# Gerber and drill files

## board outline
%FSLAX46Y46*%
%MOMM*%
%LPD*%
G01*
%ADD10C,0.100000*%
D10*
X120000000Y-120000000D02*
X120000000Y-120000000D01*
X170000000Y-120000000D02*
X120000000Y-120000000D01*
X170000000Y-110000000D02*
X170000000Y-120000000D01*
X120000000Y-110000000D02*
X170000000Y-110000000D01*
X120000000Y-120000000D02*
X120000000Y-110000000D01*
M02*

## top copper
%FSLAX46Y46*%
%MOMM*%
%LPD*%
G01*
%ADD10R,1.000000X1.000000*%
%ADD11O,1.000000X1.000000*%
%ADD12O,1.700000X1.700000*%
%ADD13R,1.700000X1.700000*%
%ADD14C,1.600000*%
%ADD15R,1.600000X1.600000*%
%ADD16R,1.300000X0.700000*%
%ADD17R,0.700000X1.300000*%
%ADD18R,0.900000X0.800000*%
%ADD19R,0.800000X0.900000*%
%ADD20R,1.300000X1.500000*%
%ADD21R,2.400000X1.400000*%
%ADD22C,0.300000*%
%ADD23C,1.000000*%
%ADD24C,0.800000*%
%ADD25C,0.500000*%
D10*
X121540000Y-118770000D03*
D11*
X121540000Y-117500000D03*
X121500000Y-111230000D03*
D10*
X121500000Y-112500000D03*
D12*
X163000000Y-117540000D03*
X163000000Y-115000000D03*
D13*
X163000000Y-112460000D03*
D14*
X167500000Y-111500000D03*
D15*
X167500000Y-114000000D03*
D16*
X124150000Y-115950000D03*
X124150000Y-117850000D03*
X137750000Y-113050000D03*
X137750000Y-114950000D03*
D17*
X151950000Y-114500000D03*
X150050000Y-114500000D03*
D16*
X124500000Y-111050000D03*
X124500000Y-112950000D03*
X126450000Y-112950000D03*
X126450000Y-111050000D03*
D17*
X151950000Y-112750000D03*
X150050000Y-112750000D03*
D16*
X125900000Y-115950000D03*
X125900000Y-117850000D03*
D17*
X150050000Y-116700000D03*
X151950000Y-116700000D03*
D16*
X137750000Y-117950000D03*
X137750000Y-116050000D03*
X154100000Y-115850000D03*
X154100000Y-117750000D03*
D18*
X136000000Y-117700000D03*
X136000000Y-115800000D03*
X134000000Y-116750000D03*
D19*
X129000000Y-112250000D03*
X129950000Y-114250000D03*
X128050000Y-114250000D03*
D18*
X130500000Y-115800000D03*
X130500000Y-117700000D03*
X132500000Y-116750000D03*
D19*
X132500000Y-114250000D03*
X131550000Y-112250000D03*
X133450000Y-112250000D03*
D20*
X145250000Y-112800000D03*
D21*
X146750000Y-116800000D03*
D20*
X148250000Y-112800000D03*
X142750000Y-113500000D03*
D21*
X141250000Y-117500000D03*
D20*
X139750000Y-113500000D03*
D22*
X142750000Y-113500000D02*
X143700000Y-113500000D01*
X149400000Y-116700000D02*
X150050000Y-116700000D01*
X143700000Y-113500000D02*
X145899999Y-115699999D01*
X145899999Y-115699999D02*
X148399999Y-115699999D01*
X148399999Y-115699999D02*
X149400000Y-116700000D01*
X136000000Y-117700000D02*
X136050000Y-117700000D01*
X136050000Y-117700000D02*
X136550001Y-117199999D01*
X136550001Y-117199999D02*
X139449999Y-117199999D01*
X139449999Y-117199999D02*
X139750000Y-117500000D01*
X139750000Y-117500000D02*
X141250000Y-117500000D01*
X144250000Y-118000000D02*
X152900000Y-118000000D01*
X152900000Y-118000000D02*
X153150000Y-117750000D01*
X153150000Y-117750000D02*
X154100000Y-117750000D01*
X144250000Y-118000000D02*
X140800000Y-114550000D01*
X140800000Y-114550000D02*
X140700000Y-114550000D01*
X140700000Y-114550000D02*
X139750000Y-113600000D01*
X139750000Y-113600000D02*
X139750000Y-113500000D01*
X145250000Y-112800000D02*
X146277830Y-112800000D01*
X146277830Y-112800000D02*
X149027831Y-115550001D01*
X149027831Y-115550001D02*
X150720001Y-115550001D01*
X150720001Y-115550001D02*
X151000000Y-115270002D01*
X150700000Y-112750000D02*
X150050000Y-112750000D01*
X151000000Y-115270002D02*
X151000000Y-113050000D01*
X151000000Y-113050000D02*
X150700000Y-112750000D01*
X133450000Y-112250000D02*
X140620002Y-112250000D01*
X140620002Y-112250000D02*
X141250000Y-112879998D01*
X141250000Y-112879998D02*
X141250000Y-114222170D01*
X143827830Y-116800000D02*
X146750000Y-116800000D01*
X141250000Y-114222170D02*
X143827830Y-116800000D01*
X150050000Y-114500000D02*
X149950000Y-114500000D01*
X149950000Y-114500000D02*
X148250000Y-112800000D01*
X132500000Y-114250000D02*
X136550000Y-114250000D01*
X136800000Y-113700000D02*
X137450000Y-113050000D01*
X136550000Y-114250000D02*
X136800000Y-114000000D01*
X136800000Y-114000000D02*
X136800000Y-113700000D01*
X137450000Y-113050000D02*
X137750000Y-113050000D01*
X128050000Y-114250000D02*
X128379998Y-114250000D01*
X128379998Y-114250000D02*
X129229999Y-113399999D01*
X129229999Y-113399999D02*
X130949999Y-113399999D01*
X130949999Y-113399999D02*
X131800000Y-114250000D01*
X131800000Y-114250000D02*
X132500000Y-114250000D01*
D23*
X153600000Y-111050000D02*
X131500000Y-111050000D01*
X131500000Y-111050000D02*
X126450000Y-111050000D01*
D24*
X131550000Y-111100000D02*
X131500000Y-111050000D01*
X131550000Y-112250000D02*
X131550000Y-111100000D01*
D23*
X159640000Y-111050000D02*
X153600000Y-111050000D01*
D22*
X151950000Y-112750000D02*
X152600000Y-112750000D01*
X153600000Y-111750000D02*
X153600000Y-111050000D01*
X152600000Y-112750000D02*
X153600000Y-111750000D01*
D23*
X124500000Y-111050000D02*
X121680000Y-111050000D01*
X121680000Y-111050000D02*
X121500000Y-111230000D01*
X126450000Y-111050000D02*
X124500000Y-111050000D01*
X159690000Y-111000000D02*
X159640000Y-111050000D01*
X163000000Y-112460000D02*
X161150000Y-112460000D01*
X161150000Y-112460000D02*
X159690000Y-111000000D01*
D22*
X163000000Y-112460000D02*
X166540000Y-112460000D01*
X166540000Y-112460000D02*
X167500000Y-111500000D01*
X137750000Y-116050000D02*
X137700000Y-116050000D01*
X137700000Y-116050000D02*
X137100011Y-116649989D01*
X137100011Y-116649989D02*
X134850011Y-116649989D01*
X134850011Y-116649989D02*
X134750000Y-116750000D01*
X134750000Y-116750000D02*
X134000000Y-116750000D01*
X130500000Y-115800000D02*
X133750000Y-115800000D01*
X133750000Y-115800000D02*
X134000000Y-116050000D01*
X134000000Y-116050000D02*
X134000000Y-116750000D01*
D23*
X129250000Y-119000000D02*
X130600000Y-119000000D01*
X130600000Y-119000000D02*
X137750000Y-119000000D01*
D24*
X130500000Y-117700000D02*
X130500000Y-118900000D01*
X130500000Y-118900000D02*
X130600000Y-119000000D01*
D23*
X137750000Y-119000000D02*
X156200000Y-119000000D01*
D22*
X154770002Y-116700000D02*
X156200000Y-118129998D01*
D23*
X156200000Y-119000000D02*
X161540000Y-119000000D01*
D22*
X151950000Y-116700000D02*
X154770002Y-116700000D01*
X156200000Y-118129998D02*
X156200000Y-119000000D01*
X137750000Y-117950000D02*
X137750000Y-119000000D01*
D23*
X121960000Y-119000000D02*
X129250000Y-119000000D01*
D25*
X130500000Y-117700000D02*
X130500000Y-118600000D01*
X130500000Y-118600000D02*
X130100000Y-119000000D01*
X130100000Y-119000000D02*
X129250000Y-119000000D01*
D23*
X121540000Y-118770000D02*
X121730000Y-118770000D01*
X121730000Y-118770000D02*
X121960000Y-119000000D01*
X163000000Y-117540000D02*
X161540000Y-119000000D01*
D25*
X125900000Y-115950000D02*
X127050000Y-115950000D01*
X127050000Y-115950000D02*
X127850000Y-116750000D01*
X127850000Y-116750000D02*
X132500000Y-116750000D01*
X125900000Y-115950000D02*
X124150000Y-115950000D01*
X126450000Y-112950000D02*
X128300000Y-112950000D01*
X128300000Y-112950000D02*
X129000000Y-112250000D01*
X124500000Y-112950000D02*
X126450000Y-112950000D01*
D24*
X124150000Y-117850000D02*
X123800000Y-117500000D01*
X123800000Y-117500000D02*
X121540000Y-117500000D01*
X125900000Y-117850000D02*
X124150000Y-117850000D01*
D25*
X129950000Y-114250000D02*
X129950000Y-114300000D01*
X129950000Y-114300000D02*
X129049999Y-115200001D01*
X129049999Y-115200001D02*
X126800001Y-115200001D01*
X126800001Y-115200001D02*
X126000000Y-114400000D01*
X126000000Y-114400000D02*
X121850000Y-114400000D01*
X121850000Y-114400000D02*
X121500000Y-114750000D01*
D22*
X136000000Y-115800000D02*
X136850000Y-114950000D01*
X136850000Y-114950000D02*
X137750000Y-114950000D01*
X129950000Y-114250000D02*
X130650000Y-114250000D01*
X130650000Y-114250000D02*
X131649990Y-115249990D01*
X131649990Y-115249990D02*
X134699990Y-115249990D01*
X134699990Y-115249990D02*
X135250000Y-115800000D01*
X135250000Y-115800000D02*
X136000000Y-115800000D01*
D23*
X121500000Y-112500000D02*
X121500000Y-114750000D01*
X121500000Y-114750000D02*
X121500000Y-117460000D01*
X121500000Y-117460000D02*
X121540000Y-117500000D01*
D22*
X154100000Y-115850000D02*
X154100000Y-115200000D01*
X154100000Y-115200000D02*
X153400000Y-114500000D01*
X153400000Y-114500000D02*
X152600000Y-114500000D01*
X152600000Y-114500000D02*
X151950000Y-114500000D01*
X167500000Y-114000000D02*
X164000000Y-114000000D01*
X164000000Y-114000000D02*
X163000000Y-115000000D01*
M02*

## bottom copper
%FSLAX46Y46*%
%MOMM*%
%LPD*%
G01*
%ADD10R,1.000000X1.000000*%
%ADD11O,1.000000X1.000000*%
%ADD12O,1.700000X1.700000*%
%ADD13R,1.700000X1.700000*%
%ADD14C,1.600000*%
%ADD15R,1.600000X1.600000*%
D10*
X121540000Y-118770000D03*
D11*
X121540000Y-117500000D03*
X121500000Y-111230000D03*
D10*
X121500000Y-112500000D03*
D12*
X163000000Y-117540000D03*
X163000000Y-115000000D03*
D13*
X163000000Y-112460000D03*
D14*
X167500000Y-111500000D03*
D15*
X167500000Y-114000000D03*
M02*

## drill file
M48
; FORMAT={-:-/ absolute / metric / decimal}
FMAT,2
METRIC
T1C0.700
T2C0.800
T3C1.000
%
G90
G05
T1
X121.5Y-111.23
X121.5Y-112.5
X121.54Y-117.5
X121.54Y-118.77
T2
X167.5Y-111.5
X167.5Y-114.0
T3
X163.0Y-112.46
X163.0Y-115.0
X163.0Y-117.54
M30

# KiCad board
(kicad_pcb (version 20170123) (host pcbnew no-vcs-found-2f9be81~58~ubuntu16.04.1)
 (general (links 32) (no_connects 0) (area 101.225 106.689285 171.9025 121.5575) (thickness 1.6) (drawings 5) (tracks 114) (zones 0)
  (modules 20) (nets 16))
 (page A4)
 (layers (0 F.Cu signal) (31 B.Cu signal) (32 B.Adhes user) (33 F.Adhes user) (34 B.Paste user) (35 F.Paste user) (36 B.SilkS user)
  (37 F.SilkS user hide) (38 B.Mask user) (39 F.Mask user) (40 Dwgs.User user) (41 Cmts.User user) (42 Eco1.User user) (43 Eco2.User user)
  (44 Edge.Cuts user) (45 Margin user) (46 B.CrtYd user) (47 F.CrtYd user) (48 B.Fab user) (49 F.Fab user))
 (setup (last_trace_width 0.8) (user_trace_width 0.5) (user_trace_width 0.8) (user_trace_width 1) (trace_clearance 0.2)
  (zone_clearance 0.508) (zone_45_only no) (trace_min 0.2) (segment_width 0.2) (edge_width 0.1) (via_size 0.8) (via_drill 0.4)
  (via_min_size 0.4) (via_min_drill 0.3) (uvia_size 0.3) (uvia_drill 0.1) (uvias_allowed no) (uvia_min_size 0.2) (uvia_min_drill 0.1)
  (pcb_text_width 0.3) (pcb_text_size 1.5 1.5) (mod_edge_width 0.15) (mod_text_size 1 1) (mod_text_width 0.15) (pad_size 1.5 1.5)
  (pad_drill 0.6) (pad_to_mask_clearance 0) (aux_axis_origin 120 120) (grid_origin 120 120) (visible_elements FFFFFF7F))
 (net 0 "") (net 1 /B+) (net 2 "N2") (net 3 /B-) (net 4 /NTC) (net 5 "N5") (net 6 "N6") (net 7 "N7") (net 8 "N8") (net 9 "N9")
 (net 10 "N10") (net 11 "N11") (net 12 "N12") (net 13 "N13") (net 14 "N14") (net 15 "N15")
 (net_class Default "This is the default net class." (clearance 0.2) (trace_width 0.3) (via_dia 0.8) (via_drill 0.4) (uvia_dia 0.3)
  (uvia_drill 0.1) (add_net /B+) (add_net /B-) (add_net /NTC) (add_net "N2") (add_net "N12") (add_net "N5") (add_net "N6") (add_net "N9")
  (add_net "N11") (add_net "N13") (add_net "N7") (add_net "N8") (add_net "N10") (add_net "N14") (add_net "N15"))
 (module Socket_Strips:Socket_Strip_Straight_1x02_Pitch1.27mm (layer F.Cu) (at 121.54 118.77 180)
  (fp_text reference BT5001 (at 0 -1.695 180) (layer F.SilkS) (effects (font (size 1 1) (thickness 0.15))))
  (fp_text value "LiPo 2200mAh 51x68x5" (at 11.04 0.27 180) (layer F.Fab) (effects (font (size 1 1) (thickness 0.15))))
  (pad 1 thru_hole rect (at 0 0 180) (size 1 1) (drill 0.7) (layers *.Cu *.Mask) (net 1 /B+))
  (pad 2 thru_hole oval (at 0 1.27 180) (size 1 1) (drill 0.7) (layers *.Cu *.Mask) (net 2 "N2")))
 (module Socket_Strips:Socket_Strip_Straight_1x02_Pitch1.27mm (layer F.Cu) (at 121.5 112.5 180)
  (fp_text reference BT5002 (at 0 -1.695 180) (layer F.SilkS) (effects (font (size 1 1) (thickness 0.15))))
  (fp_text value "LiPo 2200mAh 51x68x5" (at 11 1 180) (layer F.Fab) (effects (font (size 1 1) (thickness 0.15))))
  (pad 2 thru_hole oval (at 0 1.27 180) (size 1 1) (drill 0.7) (layers *.Cu *.Mask) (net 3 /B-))
  (pad 1 thru_hole rect (at 0 0 180) (size 1 1) (drill 0.7) (layers *.Cu *.Mask) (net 2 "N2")))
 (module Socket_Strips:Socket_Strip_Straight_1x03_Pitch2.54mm (layer F.Cu) (at 163 112.46)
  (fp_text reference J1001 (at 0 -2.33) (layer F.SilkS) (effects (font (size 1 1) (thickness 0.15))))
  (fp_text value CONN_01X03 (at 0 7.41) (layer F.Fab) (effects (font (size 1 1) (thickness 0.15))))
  (pad 3 thru_hole oval (at 0 5.08) (size 1.7 1.7) (drill 1) (layers *.Cu *.Mask) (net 1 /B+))
  (pad 2 thru_hole oval (at 0 2.54) (size 1.7 1.7) (drill 1) (layers *.Cu *.Mask) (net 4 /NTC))
  (pad 1 thru_hole rect (at 0 0) (size 1.7 1.7) (drill 1) (layers *.Cu *.Mask) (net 3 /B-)))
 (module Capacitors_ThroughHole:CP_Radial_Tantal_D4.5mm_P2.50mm (layer F.Cu) (at 167.5 114 90)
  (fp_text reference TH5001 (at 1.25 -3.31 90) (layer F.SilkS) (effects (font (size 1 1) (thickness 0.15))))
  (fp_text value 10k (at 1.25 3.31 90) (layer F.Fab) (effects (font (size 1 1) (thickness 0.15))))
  (pad 2 thru_hole circle (at 2.5 0 90) (size 1.6 1.6) (drill 0.8) (layers *.Cu *.Mask) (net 3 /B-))
  (pad 1 thru_hole rect (at 0 0 90) (size 1.6 1.6) (drill 0.8) (layers *.Cu *.Mask) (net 4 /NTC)))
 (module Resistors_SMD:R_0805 (layer F.Cu) (at 124.15 116.9 270)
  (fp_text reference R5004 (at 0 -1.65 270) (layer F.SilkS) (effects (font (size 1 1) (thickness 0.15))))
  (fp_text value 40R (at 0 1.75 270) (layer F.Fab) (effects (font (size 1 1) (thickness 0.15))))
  (pad 1 smd rect (at -0.95 0 270) (size 0.7 1.3) (layers F.Cu F.Paste F.Mask) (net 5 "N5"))
  (pad 2 smd rect (at 0.95 0 270) (size 0.7 1.3) (layers F.Cu F.Paste F.Mask) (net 2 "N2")))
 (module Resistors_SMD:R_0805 (layer F.Cu) (at 137.75 114 90)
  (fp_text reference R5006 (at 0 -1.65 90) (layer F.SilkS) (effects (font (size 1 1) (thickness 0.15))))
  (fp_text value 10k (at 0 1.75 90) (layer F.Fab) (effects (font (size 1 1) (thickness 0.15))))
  (pad 2 smd rect (at 0.95 0 90) (size 0.7 1.3) (layers F.Cu F.Paste F.Mask) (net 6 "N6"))
  (pad 1 smd rect (at -0.95 0 90) (size 0.7 1.3) (layers F.Cu F.Paste F.Mask) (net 2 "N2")))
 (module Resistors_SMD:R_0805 (layer F.Cu) (at 151 114.5 180)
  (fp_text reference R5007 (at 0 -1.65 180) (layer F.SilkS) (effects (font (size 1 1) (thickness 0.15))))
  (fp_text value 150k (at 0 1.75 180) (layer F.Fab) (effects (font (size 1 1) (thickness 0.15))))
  (pad 1 smd rect (at -0.95 0 180) (size 0.7 1.3) (layers F.Cu F.Paste F.Mask) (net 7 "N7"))
  (pad 2 smd rect (at 0.95 0 180) (size 0.7 1.3) (layers F.Cu F.Paste F.Mask) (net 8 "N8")))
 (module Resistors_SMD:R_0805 (layer F.Cu) (at 124.5 112 90)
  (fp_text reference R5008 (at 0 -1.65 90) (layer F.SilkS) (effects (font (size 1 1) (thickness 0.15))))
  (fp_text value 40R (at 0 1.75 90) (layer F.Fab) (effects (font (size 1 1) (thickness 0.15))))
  (pad 2 smd rect (at 0.95 0 90) (size 0.7 1.3) (layers F.Cu F.Paste F.Mask) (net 3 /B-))
  (pad 1 smd rect (at -0.95 0 90) (size 0.7 1.3) (layers F.Cu F.Paste F.Mask) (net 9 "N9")))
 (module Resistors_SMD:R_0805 (layer F.Cu) (at 126.45 112 90)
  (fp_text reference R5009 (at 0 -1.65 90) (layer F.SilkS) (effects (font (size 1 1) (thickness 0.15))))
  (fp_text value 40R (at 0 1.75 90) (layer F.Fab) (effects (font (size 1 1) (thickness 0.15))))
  (pad 1 smd rect (at -0.95 0 90) (size 0.7 1.3) (layers F.Cu F.Paste F.Mask) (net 9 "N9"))
  (pad 2 smd rect (at 0.95 0 90) (size 0.7 1.3) (layers F.Cu F.Paste F.Mask) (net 3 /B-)))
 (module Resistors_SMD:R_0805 (layer F.Cu) (at 151 112.75)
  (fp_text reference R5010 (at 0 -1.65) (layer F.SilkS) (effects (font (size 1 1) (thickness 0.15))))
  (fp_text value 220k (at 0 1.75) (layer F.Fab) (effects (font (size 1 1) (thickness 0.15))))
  (pad 2 smd rect (at 0.95 0) (size 0.7 1.3) (layers F.Cu F.Paste F.Mask) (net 3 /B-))
  (pad 1 smd rect (at -0.95 0) (size 0.7 1.3) (layers F.Cu F.Paste F.Mask) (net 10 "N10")))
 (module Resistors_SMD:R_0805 (layer F.Cu) (at 125.9 116.9 270)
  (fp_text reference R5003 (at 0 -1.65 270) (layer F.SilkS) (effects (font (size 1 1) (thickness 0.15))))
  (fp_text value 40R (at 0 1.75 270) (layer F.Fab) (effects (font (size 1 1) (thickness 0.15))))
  (pad 1 smd rect (at -0.95 0 270) (size 0.7 1.3) (layers F.Cu F.Paste F.Mask) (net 5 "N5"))
  (pad 2 smd rect (at 0.95 0 270) (size 0.7 1.3) (layers F.Cu F.Paste F.Mask) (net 2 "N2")))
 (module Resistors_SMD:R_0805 (layer F.Cu) (at 151 116.7 180)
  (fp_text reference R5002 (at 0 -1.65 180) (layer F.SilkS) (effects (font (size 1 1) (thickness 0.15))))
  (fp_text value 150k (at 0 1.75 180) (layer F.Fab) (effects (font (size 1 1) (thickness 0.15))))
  (pad 2 smd rect (at 0.95 0 180) (size 0.7 1.3) (layers F.Cu F.Paste F.Mask) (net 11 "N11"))
  (pad 1 smd rect (at -0.95 0 180) (size 0.7 1.3) (layers F.Cu F.Paste F.Mask) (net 1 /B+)))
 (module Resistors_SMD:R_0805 (layer F.Cu) (at 137.75 117 90)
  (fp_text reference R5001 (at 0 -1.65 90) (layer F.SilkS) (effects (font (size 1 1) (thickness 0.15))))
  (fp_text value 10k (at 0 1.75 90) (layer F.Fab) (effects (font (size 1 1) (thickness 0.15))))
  (pad 1 smd rect (at -0.95 0 90) (size 0.7 1.3) (layers F.Cu F.Paste F.Mask) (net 1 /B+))
  (pad 2 smd rect (at 0.95 0 90) (size 0.7 1.3) (layers F.Cu F.Paste F.Mask) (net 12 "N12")))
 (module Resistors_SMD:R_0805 (layer F.Cu) (at 154.1 116.8 90)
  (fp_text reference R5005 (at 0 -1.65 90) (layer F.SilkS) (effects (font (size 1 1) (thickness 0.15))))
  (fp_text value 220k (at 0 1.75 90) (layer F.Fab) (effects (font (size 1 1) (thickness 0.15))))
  (pad 2 smd rect (at 0.95 0 90) (size 0.7 1.3) (layers F.Cu F.Paste F.Mask) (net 7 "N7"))
  (pad 1 smd rect (at -0.95 0 90) (size 0.7 1.3) (layers F.Cu F.Paste F.Mask) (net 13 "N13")))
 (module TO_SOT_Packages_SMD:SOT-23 (layer F.Cu) (at 135 116.75 180)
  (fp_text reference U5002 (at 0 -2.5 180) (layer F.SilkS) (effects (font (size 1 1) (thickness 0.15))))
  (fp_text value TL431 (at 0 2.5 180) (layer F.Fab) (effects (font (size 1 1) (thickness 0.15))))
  (pad 1 smd rect (at -1 -0.95 180) (size 0.9 0.8) (layers F.Cu F.Paste F.Mask) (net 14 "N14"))
  (pad 2 smd rect (at -1 0.95 180) (size 0.9 0.8) (layers F.Cu F.Paste F.Mask) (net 2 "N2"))
  (pad 3 smd rect (at 1 0 180) (size 0.9 0.8) (layers F.Cu F.Paste F.Mask) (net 12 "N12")))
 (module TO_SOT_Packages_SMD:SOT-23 (layer F.Cu) (at 129 113.25 90)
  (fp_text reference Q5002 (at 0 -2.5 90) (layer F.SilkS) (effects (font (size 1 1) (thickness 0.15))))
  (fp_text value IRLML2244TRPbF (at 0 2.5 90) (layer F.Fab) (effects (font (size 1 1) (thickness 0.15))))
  (pad 3 smd rect (at 1 0 90) (size 0.9 0.8) (layers F.Cu F.Paste F.Mask) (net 9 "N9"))
  (pad 2 smd rect (at -1 0.95 90) (size 0.9 0.8) (layers F.Cu F.Paste F.Mask) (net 2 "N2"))
  (pad 1 smd rect (at -1 -0.95 90) (size 0.9 0.8) (layers F.Cu F.Paste F.Mask) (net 6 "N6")))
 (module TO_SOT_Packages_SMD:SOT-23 (layer F.Cu) (at 131.5 116.75)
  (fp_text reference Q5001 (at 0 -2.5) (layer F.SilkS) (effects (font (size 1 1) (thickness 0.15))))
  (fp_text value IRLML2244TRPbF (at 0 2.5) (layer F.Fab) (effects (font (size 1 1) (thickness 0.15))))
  (pad 1 smd rect (at -1 -0.95) (size 0.9 0.8) (layers F.Cu F.Paste F.Mask) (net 12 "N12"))
  (pad 2 smd rect (at -1 0.95) (size 0.9 0.8) (layers F.Cu F.Paste F.Mask) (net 1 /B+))
  (pad 3 smd rect (at 1 0) (size 0.9 0.8) (layers F.Cu F.Paste F.Mask) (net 5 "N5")))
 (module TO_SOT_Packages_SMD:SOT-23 (layer F.Cu) (at 132.5 113.25 270)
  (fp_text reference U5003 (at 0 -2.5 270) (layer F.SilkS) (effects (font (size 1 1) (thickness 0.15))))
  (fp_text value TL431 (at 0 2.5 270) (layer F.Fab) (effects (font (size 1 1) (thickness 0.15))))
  (pad 3 smd rect (at 1 0 270) (size 0.9 0.8) (layers F.Cu F.Paste F.Mask) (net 6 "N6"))
  (pad 2 smd rect (at -1 0.95 270) (size 0.9 0.8) (layers F.Cu F.Paste F.Mask) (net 3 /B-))
  (pad 1 smd rect (at -1 -0.95 270) (size 0.9 0.8) (layers F.Cu F.Paste F.Mask) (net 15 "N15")))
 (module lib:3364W (layer F.Cu) (at 146.75 114.8 180)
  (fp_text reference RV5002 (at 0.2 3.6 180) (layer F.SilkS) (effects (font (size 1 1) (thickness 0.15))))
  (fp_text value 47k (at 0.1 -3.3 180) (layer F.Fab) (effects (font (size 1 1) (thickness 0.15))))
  (pad 3 smd rect (at 1.5 2 180) (size 1.3 1.5) (layers F.Cu F.Paste F.Mask) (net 10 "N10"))
  (pad 2 smd rect (at 0 -2 180) (size 2.4 1.4) (layers F.Cu F.Paste F.Mask) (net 15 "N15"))
  (pad 1 smd rect (at -1.5 2 180) (size 1.3 1.5) (layers F.Cu F.Paste F.Mask) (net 8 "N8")))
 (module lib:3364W (layer F.Cu) (at 141.25 115.5 180)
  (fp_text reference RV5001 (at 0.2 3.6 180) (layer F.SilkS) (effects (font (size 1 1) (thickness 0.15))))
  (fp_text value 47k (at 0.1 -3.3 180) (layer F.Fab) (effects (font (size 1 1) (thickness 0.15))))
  (pad 1 smd rect (at -1.5 2 180) (size 1.3 1.5) (layers F.Cu F.Paste F.Mask) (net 11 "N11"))
  (pad 2 smd rect (at 0 -2 180) (size 2.4 1.4) (layers F.Cu F.Paste F.Mask) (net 14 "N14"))
  (pad 3 smd rect (at 1.5 2 180) (size 1.3 1.5) (layers F.Cu F.Paste F.Mask) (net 13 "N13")))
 (gr_line (start 120 120) (end 120 120) (layer Edge.Cuts) (width 0.1))
 (gr_line (start 170 120) (end 120 120) (layer Edge.Cuts) (width 0.1))
 (gr_line (start 170 110) (end 170 120) (layer Edge.Cuts) (width 0.1))
 (gr_line (start 120 110) (end 170 110) (layer Edge.Cuts) (width 0.1))
 (gr_line (start 120 120) (end 120 110) (layer Edge.Cuts) (width 0.1))
 (segment (start 142.75 113.5) (end 143.7 113.5) (width 0.3) (layer F.Cu) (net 11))
 (segment (start 149.4 116.7) (end 150.05 116.7) (width 0.3) (layer F.Cu) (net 11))
 (segment (start 143.7 113.5) (end 145.899999 115.699999) (width 0.3) (layer F.Cu) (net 11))
 (segment (start 145.899999 115.699999) (end 148.399999 115.699999) (width 0.3) (layer F.Cu) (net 11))
 (segment (start 148.399999 115.699999) (end 149.4 116.7) (width 0.3) (layer F.Cu) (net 11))
 (segment (start 136 117.7) (end 136.05 117.7) (width 0.3) (layer F.Cu) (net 14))
 (segment (start 136.05 117.7) (end 136.550001 117.199999) (width 0.3) (layer F.Cu) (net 14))
 (segment (start 136.550001 117.199999) (end 139.449999 117.199999) (width 0.3) (layer F.Cu) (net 14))
 (segment (start 139.449999 117.199999) (end 139.75 117.5) (width 0.3) (layer F.Cu) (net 14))
 (segment (start 139.75 117.5) (end 141.25 117.5) (width 0.3) (layer F.Cu) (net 14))
 (segment (start 144.25 118) (end 152.9 118) (width 0.3) (layer F.Cu) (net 13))
 (segment (start 152.9 118) (end 153.15 117.75) (width 0.3) (layer F.Cu) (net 13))
 (segment (start 153.15 117.75) (end 154.1 117.75) (width 0.3) (layer F.Cu) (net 13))
 (segment (start 144.25 118) (end 140.8 114.55) (width 0.3) (layer F.Cu) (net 13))
 (segment (start 140.8 114.55) (end 140.7 114.55) (width 0.3) (layer F.Cu) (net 13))
 (segment (start 140.7 114.55) (end 139.75 113.6) (width 0.3) (layer F.Cu) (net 13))
 (segment (start 139.75 113.6) (end 139.75 113.5) (width 0.3) (layer F.Cu) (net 13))
 (segment (start 145.25 112.8) (end 146.27783 112.8) (width 0.3) (layer F.Cu) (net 10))
 (segment (start 146.27783 112.8) (end 149.027831 115.550001) (width 0.3) (layer F.Cu) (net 10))
 (segment (start 149.027831 115.550001) (end 150.720001 115.550001) (width 0.3) (layer F.Cu) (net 10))
 (segment (start 150.720001 115.550001) (end 151 115.270002) (width 0.3) (layer F.Cu) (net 10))
 (segment (start 150.7 112.75) (end 150.05 112.75) (width 0.3) (layer F.Cu) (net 10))
 (segment (start 151 115.270002) (end 151 113.05) (width 0.3) (layer F.Cu) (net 10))
 (segment (start 151 113.05) (end 150.7 112.75) (width 0.3) (layer F.Cu) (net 10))
 (segment (start 133.45 112.25) (end 140.620002 112.25) (width 0.3) (layer F.Cu) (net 15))
 (segment (start 140.620002 112.25) (end 141.25 112.879998) (width 0.3) (layer F.Cu) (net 15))
 (segment (start 141.25 112.879998) (end 141.25 114.22217) (width 0.3) (layer F.Cu) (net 15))
 (segment (start 143.82783 116.8) (end 146.75 116.8) (width 0.3) (layer F.Cu) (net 15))
 (segment (start 141.25 114.22217) (end 143.82783 116.8) (width 0.3) (layer F.Cu) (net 15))
 (segment (start 150.05 114.5) (end 149.95 114.5) (width 0.3) (layer F.Cu) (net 8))
 (segment (start 149.95 114.5) (end 148.25 112.8) (width 0.3) (layer F.Cu) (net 8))
 (segment (start 132.5 114.25) (end 136.55 114.25) (width 0.3) (layer F.Cu) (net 6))
 (segment (start 136.8 113.7) (end 137.45 113.05) (width 0.3) (layer F.Cu) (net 6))
 (segment (start 136.55 114.25) (end 136.8 114) (width 0.3) (layer F.Cu) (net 6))
 (segment (start 136.8 114) (end 136.8 113.7) (width 0.3) (layer F.Cu) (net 6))
 (segment (start 137.45 113.05) (end 137.75 113.05) (width 0.3) (layer F.Cu) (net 6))
 (segment (start 128.05 114.25) (end 128.379998 114.25) (width 0.3) (layer F.Cu) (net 6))
 (segment (start 128.379998 114.25) (end 129.229999 113.399999) (width 0.3) (layer F.Cu) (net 6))
 (segment (start 129.229999 113.399999) (end 130.949999 113.399999) (width 0.3) (layer F.Cu) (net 6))
 (segment (start 130.949999 113.399999) (end 131.8 114.25) (width 0.3) (layer F.Cu) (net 6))
 (segment (start 131.8 114.25) (end 132.5 114.25) (width 0.3) (layer F.Cu) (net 6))
 (segment (start 153.6 111.05) (end 131.5 111.05) (width 1) (layer F.Cu) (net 3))
 (segment (start 131.5 111.05) (end 126.45 111.05) (width 1) (layer F.Cu) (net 3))
 (segment (start 131.55 111.1) (end 131.5 111.05) (width 0.8) (layer F.Cu) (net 3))
 (segment (start 131.55 112.25) (end 131.55 111.1) (width 0.8) (layer F.Cu) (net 3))
 (segment (start 159.64 111.05) (end 153.6 111.05) (width 1) (layer F.Cu) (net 3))
 (segment (start 151.95 112.75) (end 152.6 112.75) (width 0.3) (layer F.Cu) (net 3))
 (segment (start 153.6 111.75) (end 153.6 111.05) (width 0.3) (layer F.Cu) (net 3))
 (segment (start 152.6 112.75) (end 153.6 111.75) (width 0.3) (layer F.Cu) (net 3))
 (segment (start 124.5 111.05) (end 121.68 111.05) (width 1) (layer F.Cu) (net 3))
 (segment (start 121.68 111.05) (end 121.5 111.23) (width 1) (layer F.Cu) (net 3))
 (segment (start 126.45 111.05) (end 124.5 111.05) (width 1) (layer F.Cu) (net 3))
 (segment (start 159.69 111) (end 159.64 111.05) (width 1) (layer F.Cu) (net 3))
 (segment (start 163 112.46) (end 161.15 112.46) (width 1) (layer F.Cu) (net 3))
 (segment (start 161.15 112.46) (end 159.69 111) (width 1) (layer F.Cu) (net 3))
 (segment (start 163 112.46) (end 166.54 112.46) (width 0.3) (layer F.Cu) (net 3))
 (segment (start 166.54 112.46) (end 167.5 111.5) (width 0.3) (layer F.Cu) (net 3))
 (segment (start 137.75 116.05) (end 137.7 116.05) (width 0.3) (layer F.Cu) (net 12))
 (segment (start 137.7 116.05) (end 137.100011 116.649989) (width 0.3) (layer F.Cu) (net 12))
 (segment (start 137.100011 116.649989) (end 134.850011 116.649989) (width 0.3) (layer F.Cu) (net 12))
 (segment (start 134.850011 116.649989) (end 134.75 116.75) (width 0.3) (layer F.Cu) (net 12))
 (segment (start 134.75 116.75) (end 134 116.75) (width 0.3) (layer F.Cu) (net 12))
 (segment (start 130.5 115.8) (end 133.75 115.8) (width 0.3) (layer F.Cu) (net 12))
 (segment (start 133.75 115.8) (end 134 116.05) (width 0.3) (layer F.Cu) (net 12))
 (segment (start 134 116.05) (end 134 116.75) (width 0.3) (layer F.Cu) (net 12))
 (segment (start 129.25 119) (end 130.6 119) (width 1) (layer F.Cu) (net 1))
 (segment (start 130.6 119) (end 137.75 119) (width 1) (layer F.Cu) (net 1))
 (segment (start 130.5 117.7) (end 130.5 118.9) (width 0.8) (layer F.Cu) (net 1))
 (segment (start 130.5 118.9) (end 130.6 119) (width 0.8) (layer F.Cu) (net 1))
 (segment (start 137.75 119) (end 156.2 119) (width 1) (layer F.Cu) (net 1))
 (segment (start 154.770002 116.7) (end 156.2 118.129998) (width 0.3) (layer F.Cu) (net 1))
 (segment (start 156.2 119) (end 161.54 119) (width 1) (layer F.Cu) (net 1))
 (segment (start 151.95 116.7) (end 154.770002 116.7) (width 0.3) (layer F.Cu) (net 1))
 (segment (start 156.2 118.129998) (end 156.2 119) (width 0.3) (layer F.Cu) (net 1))
 (segment (start 137.75 117.95) (end 137.75 119) (width 0.3) (layer F.Cu) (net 1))
 (segment (start 121.96 119) (end 129.25 119) (width 1) (layer F.Cu) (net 1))
 (segment (start 130.5 117.7) (end 130.5 118.6) (width 0.5) (layer F.Cu) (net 1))
 (segment (start 130.5 118.6) (end 130.1 119) (width 0.5) (layer F.Cu) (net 1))
 (segment (start 130.1 119) (end 129.25 119) (width 0.5) (layer F.Cu) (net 1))
 (segment (start 121.54 118.77) (end 121.73 118.77) (width 1) (layer F.Cu) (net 1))
 (segment (start 121.73 118.77) (end 121.96 119) (width 1) (layer F.Cu) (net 1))
 (segment (start 163 117.54) (end 161.54 119) (width 1) (layer F.Cu) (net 1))
 (segment (start 125.9 115.95) (end 127.05 115.95) (width 0.5) (layer F.Cu) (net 5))
 (segment (start 127.05 115.95) (end 127.85 116.75) (width 0.5) (layer F.Cu) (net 5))
 (segment (start 127.85 116.75) (end 132.5 116.75) (width 0.5) (layer F.Cu) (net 5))
 (segment (start 125.9 115.95) (end 124.15 115.95) (width 0.5) (layer F.Cu) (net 5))
 (segment (start 126.45 112.95) (end 128.3 112.95) (width 0.5) (layer F.Cu) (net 9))
 (segment (start 128.3 112.95) (end 129 112.25) (width 0.5) (layer F.Cu) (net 9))
 (segment (start 124.5 112.95) (end 126.45 112.95) (width 0.5) (layer F.Cu) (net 9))
 (segment (start 124.15 117.85) (end 123.8 117.5) (width 0.8) (layer F.Cu) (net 2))
 (segment (start 123.8 117.5) (end 121.54 117.5) (width 0.8) (layer F.Cu) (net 2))
 (segment (start 125.9 117.85) (end 124.15 117.85) (width 0.8) (layer F.Cu) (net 2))
 (segment (start 129.95 114.25) (end 129.95 114.3) (width 0.5) (layer F.Cu) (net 2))
 (segment (start 129.95 114.3) (end 129.049999 115.200001) (width 0.5) (layer F.Cu) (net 2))
 (segment (start 129.049999 115.200001) (end 126.800001 115.200001) (width 0.5) (layer F.Cu) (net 2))
 (segment (start 126.800001 115.200001) (end 126 114.4) (width 0.5) (layer F.Cu) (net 2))
 (segment (start 126 114.4) (end 121.85 114.4) (width 0.5) (layer F.Cu) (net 2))
 (segment (start 121.85 114.4) (end 121.5 114.75) (width 0.5) (layer F.Cu) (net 2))
 (segment (start 136 115.8) (end 136.85 114.95) (width 0.3) (layer F.Cu) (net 2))
 (segment (start 136.85 114.95) (end 137.75 114.95) (width 0.3) (layer F.Cu) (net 2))
 (segment (start 129.95 114.25) (end 130.65 114.25) (width 0.3) (layer F.Cu) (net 2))
 (segment (start 130.65 114.25) (end 131.64999 115.24999) (width 0.3) (layer F.Cu) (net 2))
 (segment (start 131.64999 115.24999) (end 134.69999 115.24999) (width 0.3) (layer F.Cu) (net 2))
 (segment (start 134.69999 115.24999) (end 135.25 115.8) (width 0.3) (layer F.Cu) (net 2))
 (segment (start 135.25 115.8) (end 136 115.8) (width 0.3) (layer F.Cu) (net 2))
 (segment (start 121.5 112.5) (end 121.5 114.75) (width 1) (layer F.Cu) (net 2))
 (segment (start 121.5 114.75) (end 121.5 117.46) (width 1) (layer F.Cu) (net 2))
 (segment (start 121.5 117.46) (end 121.54 117.5) (width 1) (layer F.Cu) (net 2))
 (segment (start 154.1 115.85) (end 154.1 115.2) (width 0.3) (layer F.Cu) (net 7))
 (segment (start 154.1 115.2) (end 153.4 114.5) (width 0.3) (layer F.Cu) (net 7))
 (segment (start 153.4 114.5) (end 152.6 114.5) (width 0.3) (layer F.Cu) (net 7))
 (segment (start 152.6 114.5) (end 151.95 114.5) (width 0.3) (layer F.Cu) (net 7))
 (segment (start 167.5 114) (end 164 114) (width 0.3) (layer F.Cu) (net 4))
 (segment (start 164 114) (end 163 115) (width 0.3) (layer F.Cu) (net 4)))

